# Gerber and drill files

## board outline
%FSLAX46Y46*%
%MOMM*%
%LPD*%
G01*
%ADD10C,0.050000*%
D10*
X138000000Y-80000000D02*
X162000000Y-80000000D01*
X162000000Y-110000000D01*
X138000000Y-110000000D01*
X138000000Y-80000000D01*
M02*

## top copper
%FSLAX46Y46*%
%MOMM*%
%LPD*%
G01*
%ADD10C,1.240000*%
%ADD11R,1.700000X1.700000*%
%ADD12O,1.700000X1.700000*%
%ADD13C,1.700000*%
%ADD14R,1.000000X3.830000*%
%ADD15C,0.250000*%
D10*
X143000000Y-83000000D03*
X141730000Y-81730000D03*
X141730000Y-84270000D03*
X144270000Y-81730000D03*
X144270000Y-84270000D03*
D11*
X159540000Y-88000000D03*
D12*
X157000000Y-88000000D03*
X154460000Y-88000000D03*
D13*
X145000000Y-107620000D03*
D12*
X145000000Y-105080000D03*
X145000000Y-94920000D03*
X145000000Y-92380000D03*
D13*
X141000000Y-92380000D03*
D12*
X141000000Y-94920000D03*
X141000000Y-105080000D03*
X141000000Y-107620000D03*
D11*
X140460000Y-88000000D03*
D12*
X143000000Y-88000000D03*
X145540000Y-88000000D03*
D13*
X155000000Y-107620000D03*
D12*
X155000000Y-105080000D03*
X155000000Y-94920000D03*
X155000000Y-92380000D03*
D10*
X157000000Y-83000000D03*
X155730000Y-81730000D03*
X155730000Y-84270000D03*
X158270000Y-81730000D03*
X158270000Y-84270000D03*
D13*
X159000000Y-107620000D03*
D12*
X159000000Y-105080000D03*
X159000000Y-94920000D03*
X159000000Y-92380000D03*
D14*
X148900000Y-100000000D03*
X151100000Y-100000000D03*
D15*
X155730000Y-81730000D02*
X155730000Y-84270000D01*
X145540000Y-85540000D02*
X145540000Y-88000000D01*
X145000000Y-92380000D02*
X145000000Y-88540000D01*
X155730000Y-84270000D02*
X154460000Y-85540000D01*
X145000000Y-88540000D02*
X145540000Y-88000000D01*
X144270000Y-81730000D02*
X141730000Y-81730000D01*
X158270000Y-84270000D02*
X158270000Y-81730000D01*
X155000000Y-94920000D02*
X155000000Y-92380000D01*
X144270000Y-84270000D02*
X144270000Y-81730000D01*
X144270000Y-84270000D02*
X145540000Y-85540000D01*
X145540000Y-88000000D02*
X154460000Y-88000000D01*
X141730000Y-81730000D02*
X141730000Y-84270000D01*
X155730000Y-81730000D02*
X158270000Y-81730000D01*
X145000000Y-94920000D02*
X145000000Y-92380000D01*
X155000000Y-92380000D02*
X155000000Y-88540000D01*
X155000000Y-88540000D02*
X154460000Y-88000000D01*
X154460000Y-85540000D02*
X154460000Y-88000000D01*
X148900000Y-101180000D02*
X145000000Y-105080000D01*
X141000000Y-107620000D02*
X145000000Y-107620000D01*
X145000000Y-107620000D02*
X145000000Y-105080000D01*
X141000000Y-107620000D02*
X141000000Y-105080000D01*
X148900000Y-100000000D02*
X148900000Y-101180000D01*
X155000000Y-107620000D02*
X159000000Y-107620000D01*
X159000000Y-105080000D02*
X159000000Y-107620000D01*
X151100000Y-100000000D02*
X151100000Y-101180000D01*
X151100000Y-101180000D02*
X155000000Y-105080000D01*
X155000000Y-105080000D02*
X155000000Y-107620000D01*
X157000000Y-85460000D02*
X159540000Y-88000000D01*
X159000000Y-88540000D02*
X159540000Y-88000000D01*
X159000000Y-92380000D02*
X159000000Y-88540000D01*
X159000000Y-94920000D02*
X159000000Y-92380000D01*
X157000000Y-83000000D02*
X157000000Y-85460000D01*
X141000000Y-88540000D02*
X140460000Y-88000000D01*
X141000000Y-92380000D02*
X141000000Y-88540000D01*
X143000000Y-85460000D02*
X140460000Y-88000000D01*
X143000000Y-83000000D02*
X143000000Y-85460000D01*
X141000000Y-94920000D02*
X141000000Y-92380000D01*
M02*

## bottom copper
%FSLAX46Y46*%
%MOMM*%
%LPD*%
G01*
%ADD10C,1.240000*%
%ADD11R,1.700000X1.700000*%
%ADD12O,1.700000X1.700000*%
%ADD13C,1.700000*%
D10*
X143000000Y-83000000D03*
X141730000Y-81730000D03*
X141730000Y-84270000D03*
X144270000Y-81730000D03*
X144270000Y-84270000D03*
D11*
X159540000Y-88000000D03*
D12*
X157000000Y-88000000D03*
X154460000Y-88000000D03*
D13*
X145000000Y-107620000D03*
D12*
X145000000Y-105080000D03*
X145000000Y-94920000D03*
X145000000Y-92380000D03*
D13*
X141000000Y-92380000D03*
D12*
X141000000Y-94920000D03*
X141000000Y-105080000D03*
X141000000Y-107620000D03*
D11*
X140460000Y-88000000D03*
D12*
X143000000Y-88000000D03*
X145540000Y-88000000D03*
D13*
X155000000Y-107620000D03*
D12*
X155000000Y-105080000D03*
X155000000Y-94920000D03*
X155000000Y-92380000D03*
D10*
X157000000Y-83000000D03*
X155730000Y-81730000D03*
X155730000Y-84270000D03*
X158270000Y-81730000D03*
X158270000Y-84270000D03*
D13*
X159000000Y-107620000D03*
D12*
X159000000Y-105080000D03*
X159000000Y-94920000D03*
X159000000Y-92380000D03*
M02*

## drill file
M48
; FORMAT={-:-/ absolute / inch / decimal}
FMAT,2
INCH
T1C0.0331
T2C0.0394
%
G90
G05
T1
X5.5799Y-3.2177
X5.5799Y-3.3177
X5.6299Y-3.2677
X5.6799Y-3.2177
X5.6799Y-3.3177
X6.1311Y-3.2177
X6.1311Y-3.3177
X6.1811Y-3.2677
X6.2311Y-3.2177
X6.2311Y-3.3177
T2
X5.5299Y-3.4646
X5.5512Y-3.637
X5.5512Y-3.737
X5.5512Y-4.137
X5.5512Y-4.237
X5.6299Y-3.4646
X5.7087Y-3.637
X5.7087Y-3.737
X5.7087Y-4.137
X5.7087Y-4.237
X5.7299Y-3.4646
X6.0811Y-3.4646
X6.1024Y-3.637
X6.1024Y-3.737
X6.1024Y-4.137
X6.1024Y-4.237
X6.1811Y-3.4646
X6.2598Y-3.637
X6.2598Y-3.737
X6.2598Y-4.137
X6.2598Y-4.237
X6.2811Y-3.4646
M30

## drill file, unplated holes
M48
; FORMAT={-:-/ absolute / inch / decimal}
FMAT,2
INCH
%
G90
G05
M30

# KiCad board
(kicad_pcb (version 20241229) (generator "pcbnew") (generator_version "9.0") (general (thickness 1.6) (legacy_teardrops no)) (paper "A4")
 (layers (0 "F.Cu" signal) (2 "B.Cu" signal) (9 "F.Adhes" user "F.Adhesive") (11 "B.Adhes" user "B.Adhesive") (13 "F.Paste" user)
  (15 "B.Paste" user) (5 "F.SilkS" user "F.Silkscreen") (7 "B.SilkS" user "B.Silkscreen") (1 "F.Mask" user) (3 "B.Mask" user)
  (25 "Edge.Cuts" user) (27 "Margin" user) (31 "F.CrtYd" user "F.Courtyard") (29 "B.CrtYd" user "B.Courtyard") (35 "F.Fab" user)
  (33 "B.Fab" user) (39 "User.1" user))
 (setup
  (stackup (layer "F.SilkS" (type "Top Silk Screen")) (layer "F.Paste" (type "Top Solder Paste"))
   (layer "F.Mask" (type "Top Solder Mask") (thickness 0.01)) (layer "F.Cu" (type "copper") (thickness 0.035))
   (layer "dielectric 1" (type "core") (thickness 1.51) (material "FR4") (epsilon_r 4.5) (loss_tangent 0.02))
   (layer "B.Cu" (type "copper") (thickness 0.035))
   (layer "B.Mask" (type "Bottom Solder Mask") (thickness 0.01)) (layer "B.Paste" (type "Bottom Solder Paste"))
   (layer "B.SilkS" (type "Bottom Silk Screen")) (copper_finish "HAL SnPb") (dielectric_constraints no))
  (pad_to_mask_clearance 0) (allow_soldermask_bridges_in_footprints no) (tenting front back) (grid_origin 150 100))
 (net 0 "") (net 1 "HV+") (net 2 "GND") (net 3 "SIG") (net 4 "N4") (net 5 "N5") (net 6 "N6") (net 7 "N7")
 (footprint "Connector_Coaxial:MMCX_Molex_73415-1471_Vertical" (layer "F.Cu") (at 143 83)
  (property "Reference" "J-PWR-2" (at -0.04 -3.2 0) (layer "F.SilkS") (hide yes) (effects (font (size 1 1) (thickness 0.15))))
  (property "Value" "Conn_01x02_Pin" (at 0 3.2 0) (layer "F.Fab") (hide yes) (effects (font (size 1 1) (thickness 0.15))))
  (pad "1" thru_hole circle (at 0 0) (size 1.24 1.24) (drill 0.84) (layers "*.Cu" "*.Mask") (remove_unused_layers no) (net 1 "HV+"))
  (pad "2" thru_hole circle (at -1.27 -1.27) (size 1.24 1.24) (drill 0.84) (layers "*.Cu" "*.Mask") (remove_unused_layers no) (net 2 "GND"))
  (pad "2" thru_hole circle (at -1.27 1.27) (size 1.24 1.24) (drill 0.84) (layers "*.Cu" "*.Mask") (remove_unused_layers no) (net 2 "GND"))
  (pad "2" thru_hole circle (at 1.27 -1.27) (size 1.24 1.24) (drill 0.84) (layers "*.Cu" "*.Mask") (remove_unused_layers no) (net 2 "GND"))
  (pad "2" thru_hole circle (at 1.27 1.27) (size 1.24 1.24) (drill 0.84) (layers "*.Cu" "*.Mask") (remove_unused_layers no) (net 2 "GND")))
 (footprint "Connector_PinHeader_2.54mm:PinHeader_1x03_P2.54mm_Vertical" (layer "F.Cu") (at 159.54 88 -90)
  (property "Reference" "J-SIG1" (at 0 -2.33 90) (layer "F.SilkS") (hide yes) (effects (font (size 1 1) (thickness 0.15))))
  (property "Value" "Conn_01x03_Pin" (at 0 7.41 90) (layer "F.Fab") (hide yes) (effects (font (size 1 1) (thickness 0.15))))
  (pad "1" thru_hole rect (at 0 0 270) (size 1.7 1.7) (drill 1) (layers "*.Cu" "*.Mask") (remove_unused_layers no) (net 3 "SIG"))
  (pad "2" thru_hole oval (at 0 2.54 270) (size 1.7 1.7) (drill 1) (layers "*.Cu" "*.Mask") (remove_unused_layers no) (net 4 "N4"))
  (pad "3" thru_hole oval (at 0 5.08 270) (size 1.7 1.7) (drill 1) (layers "*.Cu" "*.Mask") (remove_unused_layers no) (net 2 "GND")))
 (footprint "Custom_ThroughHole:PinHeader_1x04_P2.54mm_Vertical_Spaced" (layer "F.Cu") (at 145 100 180)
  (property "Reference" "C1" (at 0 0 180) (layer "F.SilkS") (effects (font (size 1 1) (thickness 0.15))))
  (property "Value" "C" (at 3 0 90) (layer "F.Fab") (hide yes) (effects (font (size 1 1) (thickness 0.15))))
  (pad "1" thru_hole circle (at 0 -7.62 180) (size 1.7 1.7) (drill 1) (layers "*.Cu" "*.Mask") (remove_unused_layers no) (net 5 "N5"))
  (pad "1" thru_hole oval (at 0 -5.08 180) (size 1.7 1.7) (drill 1) (layers "*.Cu" "*.Mask") (remove_unused_layers no) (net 5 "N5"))
  (pad "2" thru_hole oval (at 0 5.08 180) (size 1.7 1.7) (drill 1) (layers "*.Cu" "*.Mask") (remove_unused_layers no) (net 2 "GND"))
  (pad "2" thru_hole oval (at 0 7.62 180) (size 1.7 1.7) (drill 1) (layers "*.Cu" "*.Mask") (remove_unused_layers no) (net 2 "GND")))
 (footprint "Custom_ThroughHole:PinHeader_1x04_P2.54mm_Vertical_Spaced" (layer "F.Cu") (at 141 100)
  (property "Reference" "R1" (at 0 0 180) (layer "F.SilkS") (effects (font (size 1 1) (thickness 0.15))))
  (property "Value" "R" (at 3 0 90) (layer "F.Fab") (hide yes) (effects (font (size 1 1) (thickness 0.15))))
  (pad "1" thru_hole circle (at 0 -7.62) (size 1.7 1.7) (drill 1) (layers "*.Cu" "*.Mask") (remove_unused_layers no) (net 1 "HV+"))
  (pad "1" thru_hole oval (at 0 -5.08) (size 1.7 1.7) (drill 1) (layers "*.Cu" "*.Mask") (remove_unused_layers no) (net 1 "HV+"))
  (pad "2" thru_hole oval (at 0 5.08) (size 1.7 1.7) (drill 1) (layers "*.Cu" "*.Mask") (remove_unused_layers no) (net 5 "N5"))
  (pad "2" thru_hole oval (at 0 7.62) (size 1.7 1.7) (drill 1) (layers "*.Cu" "*.Mask") (remove_unused_layers no) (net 5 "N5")))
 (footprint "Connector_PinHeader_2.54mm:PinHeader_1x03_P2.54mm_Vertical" (layer "F.Cu") (at 140.46 88 90)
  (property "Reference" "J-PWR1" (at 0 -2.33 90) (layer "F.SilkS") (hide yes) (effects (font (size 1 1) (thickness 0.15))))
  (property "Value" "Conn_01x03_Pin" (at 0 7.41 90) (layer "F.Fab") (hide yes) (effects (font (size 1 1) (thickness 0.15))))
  (pad "1" thru_hole rect (at 0 0 90) (size 1.7 1.7) (drill 1) (layers "*.Cu" "*.Mask") (remove_unused_layers no) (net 1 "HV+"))
  (pad "2" thru_hole oval (at 0 2.54 90) (size 1.7 1.7) (drill 1) (layers "*.Cu" "*.Mask") (remove_unused_layers no) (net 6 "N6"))
  (pad "3" thru_hole oval (at 0 5.08 90) (size 1.7 1.7) (drill 1) (layers "*.Cu" "*.Mask") (remove_unused_layers no) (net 2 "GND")))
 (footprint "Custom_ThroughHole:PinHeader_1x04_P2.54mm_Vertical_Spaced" (layer "F.Cu") (at 155 100 180)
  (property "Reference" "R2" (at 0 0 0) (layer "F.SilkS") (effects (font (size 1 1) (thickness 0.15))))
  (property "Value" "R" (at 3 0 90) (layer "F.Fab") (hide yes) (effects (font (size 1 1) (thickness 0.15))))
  (pad "1" thru_hole circle (at 0 -7.62 180) (size 1.7 1.7) (drill 1) (layers "*.Cu" "*.Mask") (remove_unused_layers no) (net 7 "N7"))
  (pad "1" thru_hole oval (at 0 -5.08 180) (size 1.7 1.7) (drill 1) (layers "*.Cu" "*.Mask") (remove_unused_layers no) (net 7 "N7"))
  (pad "2" thru_hole oval (at 0 5.08 180) (size 1.7 1.7) (drill 1) (layers "*.Cu" "*.Mask") (remove_unused_layers no) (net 2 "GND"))
  (pad "2" thru_hole oval (at 0 7.62 180) (size 1.7 1.7) (drill 1) (layers "*.Cu" "*.Mask") (remove_unused_layers no) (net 2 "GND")))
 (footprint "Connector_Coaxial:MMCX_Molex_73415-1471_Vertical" (layer "F.Cu") (at 157 83)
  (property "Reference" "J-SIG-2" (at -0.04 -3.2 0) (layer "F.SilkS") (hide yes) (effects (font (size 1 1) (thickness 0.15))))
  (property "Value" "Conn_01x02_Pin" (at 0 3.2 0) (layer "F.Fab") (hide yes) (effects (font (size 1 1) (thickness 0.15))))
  (pad "1" thru_hole circle (at 0 0) (size 1.24 1.24) (drill 0.84) (layers "*.Cu" "*.Mask") (remove_unused_layers no) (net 3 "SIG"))
  (pad "2" thru_hole circle (at -1.27 -1.27) (size 1.24 1.24) (drill 0.84) (layers "*.Cu" "*.Mask") (remove_unused_layers no) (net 2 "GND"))
  (pad "2" thru_hole circle (at -1.27 1.27) (size 1.24 1.24) (drill 0.84) (layers "*.Cu" "*.Mask") (remove_unused_layers no) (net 2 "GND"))
  (pad "2" thru_hole circle (at 1.27 -1.27) (size 1.24 1.24) (drill 0.84) (layers "*.Cu" "*.Mask") (remove_unused_layers no) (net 2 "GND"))
  (pad "2" thru_hole circle (at 1.27 1.27) (size 1.24 1.24) (drill 0.84) (layers "*.Cu" "*.Mask") (remove_unused_layers no) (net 2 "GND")))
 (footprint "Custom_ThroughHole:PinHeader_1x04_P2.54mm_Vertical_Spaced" (layer "F.Cu") (at 159 100 180)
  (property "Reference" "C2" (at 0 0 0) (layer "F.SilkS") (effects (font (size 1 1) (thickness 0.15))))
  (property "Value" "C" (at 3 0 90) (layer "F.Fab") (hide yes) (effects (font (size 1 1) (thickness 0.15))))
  (pad "1" thru_hole circle (at 0 -7.62 180) (size 1.7 1.7) (drill 1) (layers "*.Cu" "*.Mask") (remove_unused_layers no) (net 7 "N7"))
  (pad "1" thru_hole oval (at 0 -5.08 180) (size 1.7 1.7) (drill 1) (layers "*.Cu" "*.Mask") (remove_unused_layers no) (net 7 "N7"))
  (pad "2" thru_hole oval (at 0 5.08 180) (size 1.7 1.7) (drill 1) (layers "*.Cu" "*.Mask") (remove_unused_layers no) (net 3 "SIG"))
  (pad "2" thru_hole oval (at 0 7.62 180) (size 1.7 1.7) (drill 1) (layers "*.Cu" "*.Mask") (remove_unused_layers no) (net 3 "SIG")))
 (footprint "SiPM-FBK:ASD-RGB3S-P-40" (layer "F.Cu") (at 150 100)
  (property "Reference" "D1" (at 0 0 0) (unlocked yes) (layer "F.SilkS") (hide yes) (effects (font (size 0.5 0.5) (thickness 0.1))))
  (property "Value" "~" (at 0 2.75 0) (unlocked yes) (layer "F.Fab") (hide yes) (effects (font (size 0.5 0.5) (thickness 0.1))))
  (pad "1" smd rect (at -1.1 0) (size 1 3.83) (layers "F.Cu" "F.Mask" "F.Paste") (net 5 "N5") (thermal_bridge_angle 45))
  (pad "2" smd rect (at 1.1 0) (size 1 3.83) (layers "F.Cu" "F.Mask" "F.Paste") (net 7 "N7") (thermal_bridge_angle 45)))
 (gr_rect (start 138 80) (end 162 110) (stroke (width 0.05) (type default)) (fill no) (layer "Edge.Cuts"))
 (segment (start 155.73 81.73) (end 155.73 84.27) (width 0.25) (layer "F.Cu") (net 2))
 (segment (start 145.54 85.54) (end 145.54 88) (width 0.25) (layer "F.Cu") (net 2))
 (segment (start 145 92.38) (end 145 88.54) (width 0.25) (layer "F.Cu") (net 2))
 (segment (start 155.73 84.27) (end 154.46 85.54) (width 0.25) (layer "F.Cu") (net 2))
 (segment (start 145 88.54) (end 145.54 88) (width 0.25) (layer "F.Cu") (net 2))
 (segment (start 144.27 81.73) (end 141.73 81.73) (width 0.25) (layer "F.Cu") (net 2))
 (segment (start 158.27 84.27) (end 158.27 81.73) (width 0.25) (layer "F.Cu") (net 2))
 (segment (start 155 94.92) (end 155 92.38) (width 0.25) (layer "F.Cu") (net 2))
 (segment (start 144.27 84.27) (end 144.27 81.73) (width 0.25) (layer "F.Cu") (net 2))
 (segment (start 144.27 84.27) (end 145.54 85.54) (width 0.25) (layer "F.Cu") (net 2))
 (segment (start 145.54 88) (end 154.46 88) (width 0.25) (layer "F.Cu") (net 2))
 (segment (start 141.73 81.73) (end 141.73 84.27) (width 0.25) (layer "F.Cu") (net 2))
 (segment (start 155.73 81.73) (end 158.27 81.73) (width 0.25) (layer "F.Cu") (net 2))
 (segment (start 145 94.92) (end 145 92.38) (width 0.25) (layer "F.Cu") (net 2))
 (segment (start 155 92.38) (end 155 88.54) (width 0.25) (layer "F.Cu") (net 2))
 (segment (start 155 88.54) (end 154.46 88) (width 0.25) (layer "F.Cu") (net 2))
 (segment (start 154.46 85.54) (end 154.46 88) (width 0.25) (layer "F.Cu") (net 2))
 (segment (start 148.9 101.18) (end 145 105.08) (width 0.25) (layer "F.Cu") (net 5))
 (segment (start 141 107.62) (end 145 107.62) (width 0.25) (layer "F.Cu") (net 5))
 (segment (start 145 107.62) (end 145 105.08) (width 0.25) (layer "F.Cu") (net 5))
 (segment (start 141 107.62) (end 141 105.08) (width 0.25) (layer "F.Cu") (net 5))
 (segment (start 148.9 100) (end 148.9 101.18) (width 0.25) (layer "F.Cu") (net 5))
 (segment (start 155 107.62) (end 159 107.62) (width 0.25) (layer "F.Cu") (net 7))
 (segment (start 159 105.08) (end 159 107.62) (width 0.25) (layer "F.Cu") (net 7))
 (segment (start 151.1 100) (end 151.1 101.18) (width 0.25) (layer "F.Cu") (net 7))
 (segment (start 151.1 101.18) (end 155 105.08) (width 0.25) (layer "F.Cu") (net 7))
 (segment (start 155 105.08) (end 155 107.62) (width 0.25) (layer "F.Cu") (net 7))
 (segment (start 157 85.46) (end 159.54 88) (width 0.25) (layer "F.Cu") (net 3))
 (segment (start 159 88.54) (end 159.54 88) (width 0.25) (layer "F.Cu") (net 3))
 (segment (start 159 92.38) (end 159 88.54) (width 0.25) (layer "F.Cu") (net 3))
 (segment (start 159 94.92) (end 159 92.38) (width 0.25) (layer "F.Cu") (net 3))
 (segment (start 157 83) (end 157 85.46) (width 0.25) (layer "F.Cu") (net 3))
 (segment (start 141 88.54) (end 140.46 88) (width 0.25) (layer "F.Cu") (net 1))
 (segment (start 141 92.38) (end 141 88.54) (width 0.25) (layer "F.Cu") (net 1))
 (segment (start 143 85.46) (end 140.46 88) (width 0.25) (layer "F.Cu") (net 1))
 (segment (start 143 83) (end 143 85.46) (width 0.25) (layer "F.Cu") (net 1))
 (segment (start 141 94.92) (end 141 92.38) (width 0.25) (layer "F.Cu") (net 1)))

